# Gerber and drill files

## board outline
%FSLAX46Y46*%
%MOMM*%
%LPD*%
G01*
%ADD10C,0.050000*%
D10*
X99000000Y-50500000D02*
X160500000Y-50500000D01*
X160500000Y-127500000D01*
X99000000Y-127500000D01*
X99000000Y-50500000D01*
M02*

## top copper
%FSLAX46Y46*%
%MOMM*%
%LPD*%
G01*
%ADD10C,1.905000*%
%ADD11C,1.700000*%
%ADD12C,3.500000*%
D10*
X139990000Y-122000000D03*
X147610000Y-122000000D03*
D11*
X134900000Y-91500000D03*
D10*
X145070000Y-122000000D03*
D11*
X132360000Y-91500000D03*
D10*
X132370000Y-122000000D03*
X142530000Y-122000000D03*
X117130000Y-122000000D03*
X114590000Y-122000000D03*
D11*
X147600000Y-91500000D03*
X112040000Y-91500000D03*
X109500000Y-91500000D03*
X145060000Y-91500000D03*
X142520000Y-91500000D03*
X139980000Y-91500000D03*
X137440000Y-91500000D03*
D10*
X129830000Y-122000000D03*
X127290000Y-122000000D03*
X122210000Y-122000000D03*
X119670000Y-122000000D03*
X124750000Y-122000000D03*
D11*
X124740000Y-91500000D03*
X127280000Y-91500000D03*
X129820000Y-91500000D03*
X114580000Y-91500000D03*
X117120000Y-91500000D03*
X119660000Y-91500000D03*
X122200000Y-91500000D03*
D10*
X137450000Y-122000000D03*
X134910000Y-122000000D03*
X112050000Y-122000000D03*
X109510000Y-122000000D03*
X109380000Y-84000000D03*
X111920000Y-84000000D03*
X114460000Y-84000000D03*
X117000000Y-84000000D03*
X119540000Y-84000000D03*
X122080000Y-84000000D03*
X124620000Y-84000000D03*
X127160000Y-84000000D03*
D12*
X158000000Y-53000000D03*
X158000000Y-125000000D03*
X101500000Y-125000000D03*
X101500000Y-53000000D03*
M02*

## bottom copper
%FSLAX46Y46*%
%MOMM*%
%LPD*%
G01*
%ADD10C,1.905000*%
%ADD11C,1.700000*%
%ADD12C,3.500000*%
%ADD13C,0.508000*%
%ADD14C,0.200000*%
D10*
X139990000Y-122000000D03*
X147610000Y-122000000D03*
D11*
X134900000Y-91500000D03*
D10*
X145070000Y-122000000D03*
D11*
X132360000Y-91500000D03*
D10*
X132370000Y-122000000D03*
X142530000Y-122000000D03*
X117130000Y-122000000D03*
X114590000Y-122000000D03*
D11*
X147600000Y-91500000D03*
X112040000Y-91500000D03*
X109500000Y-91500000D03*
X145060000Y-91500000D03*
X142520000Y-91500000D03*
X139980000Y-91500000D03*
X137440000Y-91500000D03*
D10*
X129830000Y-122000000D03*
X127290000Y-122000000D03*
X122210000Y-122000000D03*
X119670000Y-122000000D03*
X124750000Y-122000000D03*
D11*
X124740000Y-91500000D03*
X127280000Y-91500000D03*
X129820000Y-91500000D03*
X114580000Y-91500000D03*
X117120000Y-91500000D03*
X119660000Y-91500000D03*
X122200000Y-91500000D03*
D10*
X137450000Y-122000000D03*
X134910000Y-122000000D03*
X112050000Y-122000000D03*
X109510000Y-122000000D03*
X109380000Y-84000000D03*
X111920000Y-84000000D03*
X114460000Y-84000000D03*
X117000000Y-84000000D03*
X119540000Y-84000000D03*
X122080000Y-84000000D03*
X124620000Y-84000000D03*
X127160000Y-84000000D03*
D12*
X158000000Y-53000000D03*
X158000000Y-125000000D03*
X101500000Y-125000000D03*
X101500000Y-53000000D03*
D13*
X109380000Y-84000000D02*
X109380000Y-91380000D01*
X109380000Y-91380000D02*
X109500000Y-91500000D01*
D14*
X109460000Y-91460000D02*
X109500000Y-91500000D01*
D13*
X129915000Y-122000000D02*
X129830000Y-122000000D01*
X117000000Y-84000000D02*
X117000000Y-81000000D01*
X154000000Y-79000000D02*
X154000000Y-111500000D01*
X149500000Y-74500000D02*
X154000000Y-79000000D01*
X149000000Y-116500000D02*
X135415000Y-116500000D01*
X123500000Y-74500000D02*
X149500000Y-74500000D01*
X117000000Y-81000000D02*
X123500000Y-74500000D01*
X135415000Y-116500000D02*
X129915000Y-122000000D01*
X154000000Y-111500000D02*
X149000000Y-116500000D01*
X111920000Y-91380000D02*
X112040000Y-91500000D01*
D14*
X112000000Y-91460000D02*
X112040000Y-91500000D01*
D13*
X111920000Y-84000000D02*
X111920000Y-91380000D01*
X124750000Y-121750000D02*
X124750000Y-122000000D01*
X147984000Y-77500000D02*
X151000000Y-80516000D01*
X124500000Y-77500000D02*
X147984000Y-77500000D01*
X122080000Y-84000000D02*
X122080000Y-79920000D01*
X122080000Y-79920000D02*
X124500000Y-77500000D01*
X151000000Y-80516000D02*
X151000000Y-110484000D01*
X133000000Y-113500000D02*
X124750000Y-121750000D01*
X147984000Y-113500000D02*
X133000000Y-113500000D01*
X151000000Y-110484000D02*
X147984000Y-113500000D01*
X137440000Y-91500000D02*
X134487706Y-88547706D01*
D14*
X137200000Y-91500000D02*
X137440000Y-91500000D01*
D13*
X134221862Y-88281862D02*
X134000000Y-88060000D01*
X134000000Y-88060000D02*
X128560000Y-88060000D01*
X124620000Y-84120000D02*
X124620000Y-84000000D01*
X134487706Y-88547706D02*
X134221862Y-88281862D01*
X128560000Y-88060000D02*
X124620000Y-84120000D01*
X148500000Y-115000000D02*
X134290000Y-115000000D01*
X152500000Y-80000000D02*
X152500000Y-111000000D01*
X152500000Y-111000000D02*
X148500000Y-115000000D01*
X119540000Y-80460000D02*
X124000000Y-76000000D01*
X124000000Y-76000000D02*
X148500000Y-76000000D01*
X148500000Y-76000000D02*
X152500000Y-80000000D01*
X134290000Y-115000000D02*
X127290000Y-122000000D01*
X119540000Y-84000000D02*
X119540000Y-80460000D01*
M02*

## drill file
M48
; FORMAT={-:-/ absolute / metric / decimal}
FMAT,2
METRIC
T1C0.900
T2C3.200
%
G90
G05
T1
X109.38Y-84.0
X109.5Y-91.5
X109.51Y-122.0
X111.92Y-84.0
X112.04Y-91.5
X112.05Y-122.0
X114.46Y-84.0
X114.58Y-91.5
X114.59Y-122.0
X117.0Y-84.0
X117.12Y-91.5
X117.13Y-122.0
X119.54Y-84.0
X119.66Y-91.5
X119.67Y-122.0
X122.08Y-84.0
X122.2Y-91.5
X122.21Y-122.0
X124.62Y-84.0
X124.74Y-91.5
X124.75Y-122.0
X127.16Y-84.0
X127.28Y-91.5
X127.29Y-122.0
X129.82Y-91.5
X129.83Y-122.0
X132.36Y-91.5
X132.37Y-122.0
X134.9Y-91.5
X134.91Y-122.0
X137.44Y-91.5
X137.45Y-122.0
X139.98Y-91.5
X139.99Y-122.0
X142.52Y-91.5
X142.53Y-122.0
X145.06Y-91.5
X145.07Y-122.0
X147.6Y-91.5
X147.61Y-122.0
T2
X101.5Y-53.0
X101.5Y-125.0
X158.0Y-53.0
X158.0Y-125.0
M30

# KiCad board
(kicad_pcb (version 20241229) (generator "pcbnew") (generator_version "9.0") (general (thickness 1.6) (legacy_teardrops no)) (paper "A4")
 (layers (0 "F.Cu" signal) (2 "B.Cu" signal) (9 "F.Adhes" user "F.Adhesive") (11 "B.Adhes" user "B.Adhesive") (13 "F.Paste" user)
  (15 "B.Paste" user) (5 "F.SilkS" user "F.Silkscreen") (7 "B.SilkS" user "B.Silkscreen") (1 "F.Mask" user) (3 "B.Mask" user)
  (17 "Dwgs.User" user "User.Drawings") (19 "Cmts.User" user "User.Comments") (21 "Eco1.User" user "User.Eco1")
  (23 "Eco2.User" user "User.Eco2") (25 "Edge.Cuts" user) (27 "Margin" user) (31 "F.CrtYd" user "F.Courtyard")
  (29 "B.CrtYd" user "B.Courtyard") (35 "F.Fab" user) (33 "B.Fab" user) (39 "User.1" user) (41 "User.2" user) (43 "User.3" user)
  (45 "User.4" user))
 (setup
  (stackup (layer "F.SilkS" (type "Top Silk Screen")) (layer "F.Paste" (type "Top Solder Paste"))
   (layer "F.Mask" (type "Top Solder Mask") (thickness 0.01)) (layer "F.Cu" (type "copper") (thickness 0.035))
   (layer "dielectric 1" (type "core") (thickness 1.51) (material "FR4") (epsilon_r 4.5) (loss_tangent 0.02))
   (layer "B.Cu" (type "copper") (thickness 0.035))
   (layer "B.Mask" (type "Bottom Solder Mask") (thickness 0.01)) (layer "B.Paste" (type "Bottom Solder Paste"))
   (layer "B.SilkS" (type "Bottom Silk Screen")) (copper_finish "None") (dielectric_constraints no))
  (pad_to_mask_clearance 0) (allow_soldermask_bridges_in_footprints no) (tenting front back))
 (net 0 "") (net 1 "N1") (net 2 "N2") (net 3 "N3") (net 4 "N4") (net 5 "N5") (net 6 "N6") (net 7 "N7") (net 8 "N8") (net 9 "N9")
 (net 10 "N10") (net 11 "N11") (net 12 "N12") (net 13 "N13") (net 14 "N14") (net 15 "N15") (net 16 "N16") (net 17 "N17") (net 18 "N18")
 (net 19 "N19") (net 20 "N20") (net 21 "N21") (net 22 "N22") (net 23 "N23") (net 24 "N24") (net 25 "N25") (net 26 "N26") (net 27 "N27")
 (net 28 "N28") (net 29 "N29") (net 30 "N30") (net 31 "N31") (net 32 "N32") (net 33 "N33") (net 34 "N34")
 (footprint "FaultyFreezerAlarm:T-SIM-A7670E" (layer "F.Cu") (at 173.81 136.75 90)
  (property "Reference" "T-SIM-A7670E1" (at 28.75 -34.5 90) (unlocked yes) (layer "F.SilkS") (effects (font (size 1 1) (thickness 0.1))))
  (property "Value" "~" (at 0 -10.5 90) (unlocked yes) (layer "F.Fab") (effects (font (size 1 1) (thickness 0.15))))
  (pad "0" thru_hole circle (at 14.75 -33.82) (size 1.905 1.905) (drill 0.9) (layers "*.Cu" "*.Mask") (remove_unused_layers no) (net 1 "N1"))
  (pad "01" thru_hole circle (at 14.75 -26.2) (size 1.905 1.905) (drill 0.9) (layers "*.Cu" "*.Mask") (remove_unused_layers no) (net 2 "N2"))
  (pad "02" thru_hole circle (at 45.25 -38.91) (size 1.7 1.7) (drill 0.9) (layers "*.Cu" "*.Mask") (remove_unused_layers no) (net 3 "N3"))
  (pad "03" thru_hole circle (at 14.75 -28.74) (size 1.905 1.905) (drill 0.9) (layers "*.Cu" "*.Mask") (remove_unused_layers no)
   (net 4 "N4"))
  (pad "04" thru_hole circle (at 45.25 -41.45) (size 1.7 1.7) (drill 0.9) (layers "*.Cu" "*.Mask") (remove_unused_layers no) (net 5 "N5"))
  (pad "05" thru_hole circle (at 14.75 -41.44) (size 1.905 1.905) (drill 0.9) (layers "*.Cu" "*.Mask") (remove_unused_layers no)
   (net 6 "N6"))
  (pad "06" thru_hole circle (at 14.75 -31.28) (size 1.905 1.905) (drill 0.9) (layers "*.Cu" "*.Mask") (remove_unused_layers no)
   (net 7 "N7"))
  (pad "07" thru_hole circle (at 14.75 -56.68) (size 1.905 1.905) (drill 0.9) (layers "*.Cu" "*.Mask") (remove_unused_layers no)
   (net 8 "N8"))
  (pad "08" thru_hole circle (at 14.75 -59.22) (size 1.905 1.905) (drill 0.9) (layers "*.Cu" "*.Mask") (remove_unused_layers no)
   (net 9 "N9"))
  (pad "09" thru_hole circle (at 45.25 -26.21) (size 1.7 1.7) (drill 0.9) (layers "*.Cu" "*.Mask") (remove_unused_layers no) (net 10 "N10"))
  (pad "10" thru_hole circle (at 45.25 -61.77) (size 1.7 1.7) (drill 0.9) (layers "*.Cu" "*.Mask") (remove_unused_layers no) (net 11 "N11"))
  (pad "11" thru_hole circle (at 45.25 -64.31) (size 1.7 1.7) (drill 0.9) (layers "*.Cu" "*.Mask") (remove_unused_layers no) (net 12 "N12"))
  (pad "12" thru_hole circle (at 45.25 -28.75) (size 1.7 1.7) (drill 0.9) (layers "*.Cu" "F.Mask") (remove_unused_layers no) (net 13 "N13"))
  (pad "13" thru_hole circle (at 45.25 -31.29) (size 1.7 1.7) (drill 0.9) (layers "*.Cu" "*.Mask") (remove_unused_layers no) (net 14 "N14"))
  (pad "14" thru_hole circle (at 45.25 -33.83) (size 1.7 1.7) (drill 0.9) (layers "*.Cu" "*.Mask") (remove_unused_layers no) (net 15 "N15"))
  (pad "15" thru_hole circle (at 45.25 -36.37) (size 1.7 1.7) (drill 0.9) (layers "*.Cu" "*.Mask") (remove_unused_layers no) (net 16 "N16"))
  (pad "18" thru_hole circle (at 14.75 -43.98) (size 1.905 1.905) (drill 0.9) (layers "*.Cu" "*.Mask") (remove_unused_layers no)
   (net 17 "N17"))
  (pad "19" thru_hole circle (at 14.75 -46.52) (size 1.905 1.905) (drill 0.9) (layers "*.Cu" "*.Mask") (remove_unused_layers no)
   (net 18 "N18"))
  (pad "21" thru_hole circle (at 14.75 -51.6) (size 1.905 1.905) (drill 0.9) (layers "*.Cu" "*.Mask") (remove_unused_layers no)
   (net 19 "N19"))
  (pad "22" thru_hole circle (at 14.75 -54.14) (size 1.905 1.905) (drill 0.9) (layers "*.Cu" "*.Mask") (remove_unused_layers no)
   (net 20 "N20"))
  (pad "23" thru_hole circle (at 14.75 -49.06) (size 1.905 1.905) (drill 0.9) (layers "*.Cu" "*.Mask") (remove_unused_layers no)
   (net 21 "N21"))
  (pad "25" thru_hole circle (at 45.25 -49.07) (size 1.7 1.7) (drill 0.9) (layers "*.Cu" "*.Mask" "Dwgs.User") (remove_unused_layers no)
   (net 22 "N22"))
  (pad "26" thru_hole circle (at 45.25 -46.53) (size 1.7 1.7) (drill 0.9) (layers "*.Cu" "*.Mask") (remove_unused_layers no) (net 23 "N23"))
  (pad "27" thru_hole circle (at 45.25 -43.99) (size 1.7 1.7) (drill 0.9) (layers "*.Cu" "*.Mask") (remove_unused_layers no) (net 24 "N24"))
  (pad "32" thru_hole circle (at 45.25 -59.23) (size 1.7 1.7) (drill 0.9) (layers "*.Cu" "*.Mask" "Dwgs.User") (remove_unused_layers no)
   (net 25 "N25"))
  (pad "33" thru_hole circle (at 45.25 -56.69) (size 1.7 1.7) (drill 0.9) (layers "*.Cu" "F.Mask") (remove_unused_layers no) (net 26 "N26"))
  (pad "34" thru_hole circle (at 45.25 -54.15) (size 1.7 1.7) (drill 0.9) (layers "*.Cu" "*.Mask") (remove_unused_layers no) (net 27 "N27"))
  (pad "35" thru_hole circle (at 45.25 -51.61) (size 1.7 1.7) (drill 0.9) (layers "*.Cu" "*.Mask") (remove_unused_layers no) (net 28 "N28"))
  (pad "36" thru_hole circle (at 14.75 -36.36) (size 1.905 1.905) (drill 0.9) (layers "*.Cu" "*.Mask") (remove_unused_layers no)
   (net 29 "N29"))
  (pad "39" thru_hole circle (at 14.75 -38.9) (size 1.905 1.905) (drill 0.9) (layers "*.Cu" "F.Mask") (remove_unused_layers no)
   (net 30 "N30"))
  (pad "RX" thru_hole circle (at 14.75 -61.76) (size 1.905 1.905) (drill 0.9) (layers "*.Cu" "*.Mask" "Dwgs.User") (remove_unused_layers no)
   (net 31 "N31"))
  (pad "TX" thru_hole circle (at 14.75 -64.3) (size 1.905 1.905) (drill 0.9) (layers "*.Cu" "*.Mask") (remove_unused_layers no)
   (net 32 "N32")))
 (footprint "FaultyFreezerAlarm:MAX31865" (layer "F.Cu") (at 118.27 84)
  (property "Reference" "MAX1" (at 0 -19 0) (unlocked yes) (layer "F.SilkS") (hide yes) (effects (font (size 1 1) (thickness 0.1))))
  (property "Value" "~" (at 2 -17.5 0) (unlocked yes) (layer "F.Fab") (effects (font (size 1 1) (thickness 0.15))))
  (pad "1" thru_hole circle (at -8.89 0) (size 1.905 1.905) (drill 0.9) (layers "*.Cu" "*.Mask") (remove_unused_layers no) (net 12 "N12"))
  (pad "2" thru_hole circle (at -6.35 0) (size 1.905 1.905) (drill 0.9) (layers "*.Cu" "*.Mask") (remove_unused_layers no) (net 11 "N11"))
  (pad "3" thru_hole circle (at -3.81 0) (size 1.905 1.905) (drill 0.9) (layers "*.Cu" "*.Mask") (remove_unused_layers no) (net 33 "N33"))
  (pad "4" thru_hole circle (at -1.27 0) (size 1.905 1.905) (drill 0.9) (layers "*.Cu" "*.Mask") (remove_unused_layers no) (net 17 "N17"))
  (pad "5" thru_hole circle (at 1.27 0) (size 1.905 1.905) (drill 0.9) (layers "*.Cu" "*.Mask") (remove_unused_layers no) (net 18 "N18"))
  (pad "6" thru_hole circle (at 3.81 0) (size 1.905 1.905) (drill 0.9) (layers "*.Cu" "*.Mask") (remove_unused_layers no) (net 21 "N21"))
  (pad "7" thru_hole circle (at 6.35 0) (size 1.905 1.905) (drill 0.9) (layers "*.Cu" "*.Mask") (remove_unused_layers no) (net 16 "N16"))
  (pad "8" thru_hole circle (at 8.89 0) (size 1.905 1.905) (drill 0.9) (layers "*.Cu" "*.Mask") (remove_unused_layers no) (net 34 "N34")))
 (gr_rect (start 99 50.5) (end 160.5 127.5) (stroke (width 0.05) (type default)) (fill no) (layer "Edge.Cuts"))
 (via (at 158 53) (size 3.5) (drill 3.2) (layers "F.Cu" "B.Cu") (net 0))
 (via (at 158 125) (size 3.5) (drill 3.2) (layers "F.Cu" "B.Cu") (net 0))
 (via (at 101.5 125) (size 3.5) (drill 3.2) (layers "F.Cu" "B.Cu") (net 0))
 (via (at 101.5 53) (size 3.5) (drill 3.2) (layers "F.Cu" "B.Cu") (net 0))
 (segment (start 109.38 84) (end 109.38 91.38) (width 0.508) (layer "B.Cu") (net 12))
 (segment (start 109.38 91.38) (end 109.5 91.5) (width 0.508) (layer "B.Cu") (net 12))
 (segment (start 109.46 91.46) (end 109.5 91.5) (width 0.2) (layer "B.Cu") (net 12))
 (segment (start 129.915 122) (end 129.83 122) (width 0.508) (layer "B.Cu") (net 17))
 (segment (start 117 84) (end 117 81) (width 0.508) (layer "B.Cu") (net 17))
 (segment (start 154 79) (end 154 111.5) (width 0.508) (layer "B.Cu") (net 17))
 (segment (start 149.5 74.5) (end 154 79) (width 0.508) (layer "B.Cu") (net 17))
 (segment (start 149 116.5) (end 135.415 116.5) (width 0.508) (layer "B.Cu") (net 17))
 (segment (start 123.5 74.5) (end 149.5 74.5) (width 0.508) (layer "B.Cu") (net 17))
 (segment (start 117 81) (end 123.5 74.5) (width 0.508) (layer "B.Cu") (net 17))
 (segment (start 135.415 116.5) (end 129.915 122) (width 0.508) (layer "B.Cu") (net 17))
 (segment (start 154 111.5) (end 149 116.5) (width 0.508) (layer "B.Cu") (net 17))
 (segment (start 111.92 91.38) (end 112.04 91.5) (width 0.508) (layer "B.Cu") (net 11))
 (segment (start 112 91.46) (end 112.04 91.5) (width 0.2) (layer "B.Cu") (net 11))
 (segment (start 111.92 84) (end 111.92 91.38) (width 0.508) (layer "B.Cu") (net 11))
 (segment (start 124.75 121.75) (end 124.75 122) (width 0.508) (layer "B.Cu") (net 21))
 (segment (start 147.984 77.5) (end 151 80.516) (width 0.508) (layer "B.Cu") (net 21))
 (segment (start 124.5 77.5) (end 147.984 77.5) (width 0.508) (layer "B.Cu") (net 21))
 (segment (start 122.08 84) (end 122.08 79.92) (width 0.508) (layer "B.Cu") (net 21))
 (segment (start 122.08 79.92) (end 124.5 77.5) (width 0.508) (layer "B.Cu") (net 21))
 (segment (start 151 80.516) (end 151 110.484) (width 0.508) (layer "B.Cu") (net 21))
 (segment (start 133 113.5) (end 124.75 121.75) (width 0.508) (layer "B.Cu") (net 21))
 (segment (start 147.984 113.5) (end 133 113.5) (width 0.508) (layer "B.Cu") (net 21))
 (segment (start 151 110.484) (end 147.984 113.5) (width 0.508) (layer "B.Cu") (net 21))
 (segment (start 137.44 91.5) (end 134.487706 88.547706) (width 0.508) (layer "B.Cu") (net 16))
 (segment (start 137.2 91.5) (end 137.44 91.5) (width 0.2) (layer "B.Cu") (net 16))
 (segment (start 134.221862 88.281862) (end 134 88.06) (width 0.508) (layer "B.Cu") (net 16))
 (segment (start 134 88.06) (end 128.56 88.06) (width 0.508) (layer "B.Cu") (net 16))
 (segment (start 124.62 84.12) (end 124.62 84) (width 0.508) (layer "B.Cu") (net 16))
 (segment (start 134.487706 88.547706) (end 134.221862 88.281862) (width 0.508) (layer "B.Cu") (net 16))
 (segment (start 128.56 88.06) (end 124.62 84.12) (width 0.508) (layer "B.Cu") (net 16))
 (segment (start 148.5 115) (end 134.29 115) (width 0.508) (layer "B.Cu") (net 18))
 (segment (start 152.5 80) (end 152.5 111) (width 0.508) (layer "B.Cu") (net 18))
 (segment (start 152.5 111) (end 148.5 115) (width 0.508) (layer "B.Cu") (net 18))
 (segment (start 119.54 80.46) (end 124 76) (width 0.508) (layer "B.Cu") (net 18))
 (segment (start 124 76) (end 148.5 76) (width 0.508) (layer "B.Cu") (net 18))
 (segment (start 148.5 76) (end 152.5 80) (width 0.508) (layer "B.Cu") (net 18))
 (segment (start 134.29 115) (end 127.29 122) (width 0.508) (layer "B.Cu") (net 18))
 (segment (start 119.54 84) (end 119.54 80.46) (width 0.508) (layer "B.Cu") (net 18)))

